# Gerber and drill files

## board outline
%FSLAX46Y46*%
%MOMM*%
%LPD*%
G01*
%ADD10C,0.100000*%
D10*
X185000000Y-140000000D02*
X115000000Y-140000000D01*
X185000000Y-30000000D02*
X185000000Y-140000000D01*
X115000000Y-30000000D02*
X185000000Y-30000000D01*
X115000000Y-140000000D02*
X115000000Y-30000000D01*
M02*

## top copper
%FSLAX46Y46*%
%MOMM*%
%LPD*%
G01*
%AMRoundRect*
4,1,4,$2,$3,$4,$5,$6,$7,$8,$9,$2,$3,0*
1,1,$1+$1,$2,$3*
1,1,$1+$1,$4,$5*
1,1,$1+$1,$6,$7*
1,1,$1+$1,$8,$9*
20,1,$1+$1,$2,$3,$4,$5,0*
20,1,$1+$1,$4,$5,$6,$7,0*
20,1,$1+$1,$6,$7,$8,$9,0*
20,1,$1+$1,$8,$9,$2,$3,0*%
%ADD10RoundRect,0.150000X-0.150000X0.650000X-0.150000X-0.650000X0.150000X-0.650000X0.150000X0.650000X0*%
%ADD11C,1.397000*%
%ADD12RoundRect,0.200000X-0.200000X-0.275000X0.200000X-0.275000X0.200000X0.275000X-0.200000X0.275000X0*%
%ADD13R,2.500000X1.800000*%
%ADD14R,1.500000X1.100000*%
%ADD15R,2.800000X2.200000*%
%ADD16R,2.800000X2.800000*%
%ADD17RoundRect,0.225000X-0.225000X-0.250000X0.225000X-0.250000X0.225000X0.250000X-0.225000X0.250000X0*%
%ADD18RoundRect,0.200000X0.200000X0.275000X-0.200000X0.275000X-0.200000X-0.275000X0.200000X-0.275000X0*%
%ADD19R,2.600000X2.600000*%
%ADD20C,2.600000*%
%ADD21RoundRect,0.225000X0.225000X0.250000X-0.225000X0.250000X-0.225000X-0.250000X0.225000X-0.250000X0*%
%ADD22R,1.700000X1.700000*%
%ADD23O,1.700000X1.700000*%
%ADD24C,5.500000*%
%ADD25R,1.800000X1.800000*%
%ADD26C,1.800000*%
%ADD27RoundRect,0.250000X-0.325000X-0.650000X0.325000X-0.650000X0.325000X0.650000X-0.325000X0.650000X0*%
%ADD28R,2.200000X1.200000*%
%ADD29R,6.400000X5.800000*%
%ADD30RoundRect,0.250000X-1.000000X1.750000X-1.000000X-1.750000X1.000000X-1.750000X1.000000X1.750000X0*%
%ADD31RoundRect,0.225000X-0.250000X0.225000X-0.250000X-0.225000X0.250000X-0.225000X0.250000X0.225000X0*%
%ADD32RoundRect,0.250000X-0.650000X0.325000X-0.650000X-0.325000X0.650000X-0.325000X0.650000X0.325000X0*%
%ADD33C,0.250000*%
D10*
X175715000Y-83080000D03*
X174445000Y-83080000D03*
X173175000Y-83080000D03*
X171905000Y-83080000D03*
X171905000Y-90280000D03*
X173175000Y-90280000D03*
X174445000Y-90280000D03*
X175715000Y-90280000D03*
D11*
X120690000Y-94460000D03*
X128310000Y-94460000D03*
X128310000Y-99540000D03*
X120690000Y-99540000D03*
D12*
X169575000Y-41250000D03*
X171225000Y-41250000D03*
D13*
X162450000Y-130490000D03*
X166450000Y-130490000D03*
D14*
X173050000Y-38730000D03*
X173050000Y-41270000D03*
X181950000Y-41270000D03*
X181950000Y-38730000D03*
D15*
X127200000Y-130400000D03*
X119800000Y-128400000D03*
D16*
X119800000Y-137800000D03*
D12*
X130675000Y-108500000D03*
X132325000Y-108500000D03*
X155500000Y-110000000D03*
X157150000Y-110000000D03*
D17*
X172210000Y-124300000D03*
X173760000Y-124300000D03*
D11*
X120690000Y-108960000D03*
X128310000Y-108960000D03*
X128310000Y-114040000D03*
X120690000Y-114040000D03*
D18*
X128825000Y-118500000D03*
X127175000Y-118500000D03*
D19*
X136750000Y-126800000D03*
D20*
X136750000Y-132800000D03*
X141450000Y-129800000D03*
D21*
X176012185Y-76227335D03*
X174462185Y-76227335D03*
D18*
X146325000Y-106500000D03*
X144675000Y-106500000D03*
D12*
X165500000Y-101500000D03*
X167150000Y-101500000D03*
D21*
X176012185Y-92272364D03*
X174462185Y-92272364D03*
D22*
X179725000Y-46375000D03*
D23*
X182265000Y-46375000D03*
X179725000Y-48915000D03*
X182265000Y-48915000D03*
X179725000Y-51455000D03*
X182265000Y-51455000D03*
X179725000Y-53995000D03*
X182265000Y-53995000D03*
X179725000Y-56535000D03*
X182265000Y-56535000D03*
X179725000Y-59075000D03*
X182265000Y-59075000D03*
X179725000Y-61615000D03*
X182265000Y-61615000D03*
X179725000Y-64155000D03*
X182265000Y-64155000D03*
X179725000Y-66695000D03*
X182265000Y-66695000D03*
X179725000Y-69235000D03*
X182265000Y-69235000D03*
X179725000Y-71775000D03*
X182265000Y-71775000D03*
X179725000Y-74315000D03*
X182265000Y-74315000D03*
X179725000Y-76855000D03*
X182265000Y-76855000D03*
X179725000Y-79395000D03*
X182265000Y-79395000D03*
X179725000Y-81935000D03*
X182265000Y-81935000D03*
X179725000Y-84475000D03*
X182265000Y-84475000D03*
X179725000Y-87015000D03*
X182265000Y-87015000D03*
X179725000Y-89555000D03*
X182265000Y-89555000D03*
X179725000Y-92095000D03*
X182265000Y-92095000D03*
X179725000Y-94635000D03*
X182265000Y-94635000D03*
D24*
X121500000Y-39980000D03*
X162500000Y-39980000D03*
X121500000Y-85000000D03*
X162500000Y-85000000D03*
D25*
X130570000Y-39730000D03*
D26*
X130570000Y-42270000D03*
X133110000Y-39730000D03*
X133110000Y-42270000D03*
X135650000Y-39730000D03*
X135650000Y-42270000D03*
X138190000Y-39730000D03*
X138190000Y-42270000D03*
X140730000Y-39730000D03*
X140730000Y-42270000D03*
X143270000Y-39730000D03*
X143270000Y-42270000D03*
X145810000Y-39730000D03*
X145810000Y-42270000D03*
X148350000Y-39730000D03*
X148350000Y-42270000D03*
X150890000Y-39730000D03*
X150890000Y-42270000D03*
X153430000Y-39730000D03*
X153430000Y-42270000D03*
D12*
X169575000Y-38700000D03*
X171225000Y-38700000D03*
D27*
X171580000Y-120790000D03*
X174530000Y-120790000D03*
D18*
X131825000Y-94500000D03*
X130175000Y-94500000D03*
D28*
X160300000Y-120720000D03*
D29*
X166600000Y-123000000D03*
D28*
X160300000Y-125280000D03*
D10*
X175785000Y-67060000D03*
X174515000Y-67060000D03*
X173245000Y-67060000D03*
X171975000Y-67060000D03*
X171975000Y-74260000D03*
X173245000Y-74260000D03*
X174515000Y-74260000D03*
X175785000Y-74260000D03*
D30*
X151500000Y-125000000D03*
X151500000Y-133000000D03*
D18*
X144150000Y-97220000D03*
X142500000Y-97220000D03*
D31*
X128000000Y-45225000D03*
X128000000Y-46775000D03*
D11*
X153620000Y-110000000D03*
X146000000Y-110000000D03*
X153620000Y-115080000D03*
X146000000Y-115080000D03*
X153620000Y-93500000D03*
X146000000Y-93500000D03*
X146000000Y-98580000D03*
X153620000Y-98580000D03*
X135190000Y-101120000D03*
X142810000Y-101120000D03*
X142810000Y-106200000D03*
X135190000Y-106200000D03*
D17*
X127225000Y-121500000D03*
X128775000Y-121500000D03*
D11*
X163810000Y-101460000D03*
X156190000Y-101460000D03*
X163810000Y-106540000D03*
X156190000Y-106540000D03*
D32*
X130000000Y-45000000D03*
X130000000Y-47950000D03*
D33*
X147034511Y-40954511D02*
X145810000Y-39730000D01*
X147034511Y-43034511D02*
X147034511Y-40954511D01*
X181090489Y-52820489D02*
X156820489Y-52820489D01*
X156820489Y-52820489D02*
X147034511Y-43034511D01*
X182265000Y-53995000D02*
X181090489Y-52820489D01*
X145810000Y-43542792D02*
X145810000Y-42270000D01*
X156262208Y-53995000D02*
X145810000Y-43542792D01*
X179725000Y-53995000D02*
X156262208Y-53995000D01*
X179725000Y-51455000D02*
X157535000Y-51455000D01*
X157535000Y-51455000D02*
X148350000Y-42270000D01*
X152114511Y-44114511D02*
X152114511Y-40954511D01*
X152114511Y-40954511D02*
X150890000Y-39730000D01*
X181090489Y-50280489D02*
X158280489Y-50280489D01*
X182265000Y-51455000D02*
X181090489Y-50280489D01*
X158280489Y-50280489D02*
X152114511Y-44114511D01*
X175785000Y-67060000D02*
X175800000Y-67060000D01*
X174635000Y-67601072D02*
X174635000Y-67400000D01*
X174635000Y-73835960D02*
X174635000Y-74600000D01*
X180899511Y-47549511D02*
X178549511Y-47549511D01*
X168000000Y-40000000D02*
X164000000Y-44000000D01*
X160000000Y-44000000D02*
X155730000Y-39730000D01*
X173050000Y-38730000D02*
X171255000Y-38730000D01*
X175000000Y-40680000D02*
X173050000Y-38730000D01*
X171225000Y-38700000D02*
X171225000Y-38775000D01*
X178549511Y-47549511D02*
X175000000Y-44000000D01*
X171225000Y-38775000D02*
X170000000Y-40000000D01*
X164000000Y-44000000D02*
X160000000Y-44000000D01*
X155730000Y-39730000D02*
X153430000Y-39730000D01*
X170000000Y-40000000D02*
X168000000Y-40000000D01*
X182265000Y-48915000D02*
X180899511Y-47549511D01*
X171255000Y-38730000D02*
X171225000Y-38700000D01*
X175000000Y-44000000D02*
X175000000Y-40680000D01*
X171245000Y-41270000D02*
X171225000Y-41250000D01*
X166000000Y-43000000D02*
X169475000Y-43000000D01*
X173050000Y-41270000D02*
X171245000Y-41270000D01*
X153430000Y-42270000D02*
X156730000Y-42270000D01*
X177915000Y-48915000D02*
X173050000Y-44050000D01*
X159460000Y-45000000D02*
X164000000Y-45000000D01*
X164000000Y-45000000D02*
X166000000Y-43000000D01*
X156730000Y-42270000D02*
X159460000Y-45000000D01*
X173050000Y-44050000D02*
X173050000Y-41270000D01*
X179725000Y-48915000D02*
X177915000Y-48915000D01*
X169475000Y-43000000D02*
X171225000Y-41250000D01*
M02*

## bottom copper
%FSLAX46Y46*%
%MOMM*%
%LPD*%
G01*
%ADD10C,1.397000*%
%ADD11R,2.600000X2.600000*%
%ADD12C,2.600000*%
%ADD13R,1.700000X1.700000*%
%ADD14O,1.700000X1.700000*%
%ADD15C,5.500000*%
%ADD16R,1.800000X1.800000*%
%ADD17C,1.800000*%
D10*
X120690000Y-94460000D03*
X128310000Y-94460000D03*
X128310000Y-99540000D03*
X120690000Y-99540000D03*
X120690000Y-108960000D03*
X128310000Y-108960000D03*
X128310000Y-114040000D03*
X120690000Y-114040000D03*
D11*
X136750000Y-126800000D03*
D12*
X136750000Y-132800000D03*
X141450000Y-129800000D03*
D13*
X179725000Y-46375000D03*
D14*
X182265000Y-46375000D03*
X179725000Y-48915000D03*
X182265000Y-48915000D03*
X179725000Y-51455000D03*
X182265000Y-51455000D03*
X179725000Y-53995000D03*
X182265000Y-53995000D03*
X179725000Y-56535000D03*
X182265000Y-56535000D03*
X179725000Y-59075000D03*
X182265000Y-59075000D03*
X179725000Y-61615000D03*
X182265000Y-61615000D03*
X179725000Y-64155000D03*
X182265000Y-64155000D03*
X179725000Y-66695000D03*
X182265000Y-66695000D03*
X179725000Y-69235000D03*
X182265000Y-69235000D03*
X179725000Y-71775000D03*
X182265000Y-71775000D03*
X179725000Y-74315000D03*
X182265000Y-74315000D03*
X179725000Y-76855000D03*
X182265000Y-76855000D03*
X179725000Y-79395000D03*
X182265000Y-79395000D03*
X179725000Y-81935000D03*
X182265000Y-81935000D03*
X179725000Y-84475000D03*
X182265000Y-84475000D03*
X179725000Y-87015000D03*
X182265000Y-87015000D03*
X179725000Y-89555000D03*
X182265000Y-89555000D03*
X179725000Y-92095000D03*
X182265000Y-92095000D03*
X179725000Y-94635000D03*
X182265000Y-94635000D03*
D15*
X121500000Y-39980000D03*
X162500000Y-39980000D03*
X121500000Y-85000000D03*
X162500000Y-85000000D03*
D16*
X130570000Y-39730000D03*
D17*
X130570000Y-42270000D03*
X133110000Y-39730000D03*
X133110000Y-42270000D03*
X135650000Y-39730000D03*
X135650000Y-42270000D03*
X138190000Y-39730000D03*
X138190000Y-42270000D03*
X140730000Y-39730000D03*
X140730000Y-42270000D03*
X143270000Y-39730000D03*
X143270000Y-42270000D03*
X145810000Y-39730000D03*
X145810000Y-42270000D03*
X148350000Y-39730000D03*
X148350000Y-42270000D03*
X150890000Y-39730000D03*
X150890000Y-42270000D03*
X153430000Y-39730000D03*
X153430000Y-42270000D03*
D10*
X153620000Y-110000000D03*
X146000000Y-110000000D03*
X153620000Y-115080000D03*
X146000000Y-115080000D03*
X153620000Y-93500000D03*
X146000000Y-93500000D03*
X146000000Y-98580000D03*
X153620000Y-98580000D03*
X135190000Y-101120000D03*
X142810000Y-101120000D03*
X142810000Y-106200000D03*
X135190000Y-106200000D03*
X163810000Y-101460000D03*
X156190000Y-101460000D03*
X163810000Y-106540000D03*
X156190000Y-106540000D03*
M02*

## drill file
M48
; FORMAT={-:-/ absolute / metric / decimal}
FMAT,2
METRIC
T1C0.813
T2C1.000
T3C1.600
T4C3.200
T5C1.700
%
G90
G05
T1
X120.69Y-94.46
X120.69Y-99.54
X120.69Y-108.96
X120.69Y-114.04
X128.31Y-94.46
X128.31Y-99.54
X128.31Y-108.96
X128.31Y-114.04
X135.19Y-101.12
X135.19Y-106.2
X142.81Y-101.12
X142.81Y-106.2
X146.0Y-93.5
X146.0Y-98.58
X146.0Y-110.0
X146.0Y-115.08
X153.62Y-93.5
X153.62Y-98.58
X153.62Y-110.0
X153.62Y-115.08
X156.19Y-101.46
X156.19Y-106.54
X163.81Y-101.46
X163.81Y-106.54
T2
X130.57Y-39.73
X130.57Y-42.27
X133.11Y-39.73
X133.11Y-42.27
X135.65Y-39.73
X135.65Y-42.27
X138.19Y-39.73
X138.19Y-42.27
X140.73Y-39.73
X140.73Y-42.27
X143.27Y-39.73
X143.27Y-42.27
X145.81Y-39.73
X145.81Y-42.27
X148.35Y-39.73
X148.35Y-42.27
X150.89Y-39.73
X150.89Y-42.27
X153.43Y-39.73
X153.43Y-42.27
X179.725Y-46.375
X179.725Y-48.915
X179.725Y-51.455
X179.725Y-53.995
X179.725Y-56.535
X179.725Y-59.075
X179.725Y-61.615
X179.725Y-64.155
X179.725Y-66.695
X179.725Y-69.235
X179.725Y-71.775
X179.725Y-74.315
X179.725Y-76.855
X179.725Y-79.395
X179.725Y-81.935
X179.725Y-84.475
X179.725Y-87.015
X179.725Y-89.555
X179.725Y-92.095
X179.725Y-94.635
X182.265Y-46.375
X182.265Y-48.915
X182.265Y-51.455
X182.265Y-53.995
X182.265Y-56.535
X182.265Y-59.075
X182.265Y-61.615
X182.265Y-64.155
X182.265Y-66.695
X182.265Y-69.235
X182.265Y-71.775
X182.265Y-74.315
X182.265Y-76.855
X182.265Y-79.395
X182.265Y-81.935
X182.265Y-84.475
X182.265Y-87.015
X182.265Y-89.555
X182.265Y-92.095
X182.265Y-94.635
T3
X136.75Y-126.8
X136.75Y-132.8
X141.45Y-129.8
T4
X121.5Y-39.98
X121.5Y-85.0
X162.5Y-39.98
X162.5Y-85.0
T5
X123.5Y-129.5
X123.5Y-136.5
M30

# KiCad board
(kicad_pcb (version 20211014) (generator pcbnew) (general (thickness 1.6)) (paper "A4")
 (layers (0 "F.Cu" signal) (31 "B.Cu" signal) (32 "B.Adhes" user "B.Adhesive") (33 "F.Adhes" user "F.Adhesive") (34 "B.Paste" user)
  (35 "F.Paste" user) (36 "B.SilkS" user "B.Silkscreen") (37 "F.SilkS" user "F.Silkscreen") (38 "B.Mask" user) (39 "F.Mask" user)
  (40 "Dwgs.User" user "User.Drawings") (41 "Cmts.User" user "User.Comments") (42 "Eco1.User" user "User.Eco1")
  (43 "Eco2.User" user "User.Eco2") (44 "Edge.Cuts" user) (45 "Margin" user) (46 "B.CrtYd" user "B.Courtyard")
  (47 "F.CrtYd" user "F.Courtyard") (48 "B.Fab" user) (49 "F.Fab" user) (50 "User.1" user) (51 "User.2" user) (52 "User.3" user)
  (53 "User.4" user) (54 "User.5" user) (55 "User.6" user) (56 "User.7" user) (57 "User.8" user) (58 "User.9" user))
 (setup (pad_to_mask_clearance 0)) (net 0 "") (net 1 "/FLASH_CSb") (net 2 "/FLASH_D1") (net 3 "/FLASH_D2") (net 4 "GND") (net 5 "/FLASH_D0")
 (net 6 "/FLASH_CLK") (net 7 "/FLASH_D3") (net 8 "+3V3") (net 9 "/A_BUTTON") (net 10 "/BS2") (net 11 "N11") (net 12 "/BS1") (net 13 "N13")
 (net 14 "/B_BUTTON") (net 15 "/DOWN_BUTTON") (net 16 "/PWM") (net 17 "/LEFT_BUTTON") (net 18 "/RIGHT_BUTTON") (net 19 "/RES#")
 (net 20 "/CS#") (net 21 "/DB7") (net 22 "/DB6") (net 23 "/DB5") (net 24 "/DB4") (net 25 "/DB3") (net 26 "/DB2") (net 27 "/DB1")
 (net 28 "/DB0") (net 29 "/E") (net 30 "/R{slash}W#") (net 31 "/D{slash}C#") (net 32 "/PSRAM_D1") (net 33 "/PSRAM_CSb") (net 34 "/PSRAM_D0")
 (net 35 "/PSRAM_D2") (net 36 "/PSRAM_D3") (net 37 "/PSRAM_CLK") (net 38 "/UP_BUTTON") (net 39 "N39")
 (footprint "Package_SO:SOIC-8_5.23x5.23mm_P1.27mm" (layer "F.Cu") (at 173.81 86.68 -90)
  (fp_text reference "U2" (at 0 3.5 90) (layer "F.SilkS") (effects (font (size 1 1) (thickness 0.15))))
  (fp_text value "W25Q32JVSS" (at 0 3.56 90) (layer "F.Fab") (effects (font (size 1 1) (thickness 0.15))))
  (pad "1" smd roundrect (at -3.6 -1.905 270) (size 1.6 0.6) (layers "F.Cu" "F.Paste" "F.Mask") (roundrect_rratio 0.25) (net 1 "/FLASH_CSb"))
  (pad "2" smd roundrect (at -3.6 -0.635 270) (size 1.6 0.6) (layers "F.Cu" "F.Paste" "F.Mask") (roundrect_rratio 0.25) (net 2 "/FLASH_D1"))
  (pad "3" smd roundrect (at -3.6 0.635 270) (size 1.6 0.6) (layers "F.Cu" "F.Paste" "F.Mask") (roundrect_rratio 0.25) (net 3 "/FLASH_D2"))
  (pad "4" smd roundrect (at -3.6 1.905 270) (size 1.6 0.6) (layers "F.Cu" "F.Paste" "F.Mask") (roundrect_rratio 0.25) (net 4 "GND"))
  (pad "5" smd roundrect (at 3.6 1.905 270) (size 1.6 0.6) (layers "F.Cu" "F.Paste" "F.Mask") (roundrect_rratio 0.25) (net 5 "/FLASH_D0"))
  (pad "6" smd roundrect (at 3.6 0.635 270) (size 1.6 0.6) (layers "F.Cu" "F.Paste" "F.Mask") (roundrect_rratio 0.25) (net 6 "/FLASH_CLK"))
  (pad "7" smd roundrect (at 3.6 -0.635 270) (size 1.6 0.6) (layers "F.Cu" "F.Paste" "F.Mask") (roundrect_rratio 0.25) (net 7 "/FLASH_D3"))
  (pad "8" smd roundrect (at 3.6 -1.905 270) (size 1.6 0.6) (layers "F.Cu" "F.Paste" "F.Mask") (roundrect_rratio 0.25) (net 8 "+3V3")))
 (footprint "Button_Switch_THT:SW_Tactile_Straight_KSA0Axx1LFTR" (layer "F.Cu") (at 120.69 94.46)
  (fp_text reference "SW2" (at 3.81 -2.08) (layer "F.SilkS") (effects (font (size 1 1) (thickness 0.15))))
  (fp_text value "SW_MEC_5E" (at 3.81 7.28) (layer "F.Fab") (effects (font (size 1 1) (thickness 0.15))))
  (pad "1" thru_hole circle (at 0 0) (size 1.397 1.397) (drill 0.8128) (layers *.Cu *.Mask) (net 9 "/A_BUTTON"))
  (pad "1" thru_hole circle (at 7.62 0) (size 1.397 1.397) (drill 0.8128) (layers *.Cu *.Mask) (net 9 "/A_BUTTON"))
  (pad "2" thru_hole circle (at 7.62 5.08) (size 1.397 1.397) (drill 0.8128) (layers *.Cu *.Mask) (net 9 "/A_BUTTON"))
  (pad "2" thru_hole circle (at 0 5.08) (size 1.397 1.397) (drill 0.8128) (layers *.Cu *.Mask) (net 9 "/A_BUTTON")))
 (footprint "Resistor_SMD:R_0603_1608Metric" (layer "F.Cu") (at 170.4 41.25)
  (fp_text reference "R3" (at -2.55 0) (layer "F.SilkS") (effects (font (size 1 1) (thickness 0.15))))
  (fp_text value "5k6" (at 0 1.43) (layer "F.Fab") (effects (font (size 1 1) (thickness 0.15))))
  (pad "1" smd roundrect (at -0.825 0) (size 0.8 0.95) (layers "F.Cu" "F.Paste" "F.Mask") (roundrect_rratio 0.25) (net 4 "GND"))
  (pad "2" smd roundrect (at 0.825 0) (size 0.8 0.95) (layers "F.Cu" "F.Paste" "F.Mask") (roundrect_rratio 0.25) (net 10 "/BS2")))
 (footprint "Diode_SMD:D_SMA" (layer "F.Cu") (at 164.45 130.49)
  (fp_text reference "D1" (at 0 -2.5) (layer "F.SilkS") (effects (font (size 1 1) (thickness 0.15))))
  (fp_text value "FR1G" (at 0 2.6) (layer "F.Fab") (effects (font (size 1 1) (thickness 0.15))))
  (pad "1" smd rect (at -2 0) (size 2.5 1.8) (layers "F.Cu" "F.Paste" "F.Mask") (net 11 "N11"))
  (pad "2" smd rect (at 2 0) (size 2.5 1.8) (layers "F.Cu" "F.Paste" "F.Mask") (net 8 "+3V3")))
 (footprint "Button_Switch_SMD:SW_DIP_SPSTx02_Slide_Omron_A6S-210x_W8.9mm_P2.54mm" (layer "F.Cu") (at 177.5 40)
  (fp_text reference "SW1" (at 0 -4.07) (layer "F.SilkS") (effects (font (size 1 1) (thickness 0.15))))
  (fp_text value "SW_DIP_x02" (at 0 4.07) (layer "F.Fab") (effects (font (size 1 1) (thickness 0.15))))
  (pad "1" smd rect (at -4.45 -1.27) (size 1.5 1.1) (layers "F.Cu" "F.Paste" "F.Mask") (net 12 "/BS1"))
  (pad "2" smd rect (at -4.45 1.27) (size 1.5 1.1) (layers "F.Cu" "F.Paste" "F.Mask") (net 10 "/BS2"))
  (pad "3" smd rect (at 4.45 1.27) (size 1.5 1.1) (layers "F.Cu" "F.Paste" "F.Mask") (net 8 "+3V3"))
  (pad "4" smd rect (at 4.45 -1.27) (size 1.5 1.1) (layers "F.Cu" "F.Paste" "F.Mask") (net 8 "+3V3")))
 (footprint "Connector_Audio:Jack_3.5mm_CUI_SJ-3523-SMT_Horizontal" (layer "F.Cu") (at 123.5 132)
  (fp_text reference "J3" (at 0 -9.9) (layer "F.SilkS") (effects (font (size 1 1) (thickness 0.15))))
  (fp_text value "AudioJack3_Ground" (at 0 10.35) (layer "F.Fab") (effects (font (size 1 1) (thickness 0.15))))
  (pad "" np_thru_hole circle (at 0 4.5) (size 1.7 1.7) (drill 1.7) (layers *.Cu *.Mask))
  (pad "" np_thru_hole circle (at 0 -2.5) (size 1.7 1.7) (drill 1.7) (layers *.Cu *.Mask))
  (pad "R" smd rect (at 3.7 -1.6) (size 2.8 2.2) (layers "F.Cu" "F.Paste" "F.Mask") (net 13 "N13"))
  (pad "S" smd rect (at -3.7 -3.6) (size 2.8 2.2) (layers "F.Cu" "F.Paste" "F.Mask") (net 4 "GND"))
  (pad "T" smd rect (at -3.7 5.8) (size 2.8 2.8) (layers "F.Cu" "F.Paste" "F.Mask") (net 13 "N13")))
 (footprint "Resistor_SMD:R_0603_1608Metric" (layer "F.Cu") (at 131.5 108.5)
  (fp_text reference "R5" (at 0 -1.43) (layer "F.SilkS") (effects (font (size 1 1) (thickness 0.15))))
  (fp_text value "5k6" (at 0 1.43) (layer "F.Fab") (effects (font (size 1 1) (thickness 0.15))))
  (pad "1" smd roundrect (at -0.825 0) (size 0.8 0.95) (layers "F.Cu" "F.Paste" "F.Mask") (roundrect_rratio 0.25) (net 4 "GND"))
  (pad "2" smd roundrect (at 0.825 0) (size 0.8 0.95) (layers "F.Cu" "F.Paste" "F.Mask") (roundrect_rratio 0.25) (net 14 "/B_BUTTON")))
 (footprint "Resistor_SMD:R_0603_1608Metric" (layer "F.Cu") (at 156.325 110)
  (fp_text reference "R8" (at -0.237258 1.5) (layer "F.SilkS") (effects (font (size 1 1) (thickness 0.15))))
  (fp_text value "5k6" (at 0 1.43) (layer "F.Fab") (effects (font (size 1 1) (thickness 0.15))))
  (pad "1" smd roundrect (at -0.825 0) (size 0.8 0.95) (layers "F.Cu" "F.Paste" "F.Mask") (roundrect_rratio 0.25) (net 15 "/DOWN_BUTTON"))
  (pad "2" smd roundrect (at 0.825 0) (size 0.8 0.95) (layers "F.Cu" "F.Paste" "F.Mask") (roundrect_rratio 0.25) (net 4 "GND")))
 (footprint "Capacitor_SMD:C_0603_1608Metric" (layer "F.Cu") (at 172.985 124.3)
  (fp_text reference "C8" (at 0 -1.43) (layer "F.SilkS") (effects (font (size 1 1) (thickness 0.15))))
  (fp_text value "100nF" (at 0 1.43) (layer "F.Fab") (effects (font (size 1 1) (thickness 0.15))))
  (pad "1" smd roundrect (at -0.775 0) (size 0.9 0.95) (layers "F.Cu" "F.Paste" "F.Mask") (roundrect_rratio 0.25) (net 8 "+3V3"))
  (pad "2" smd roundrect (at 0.775 0) (size 0.9 0.95) (layers "F.Cu" "F.Paste" "F.Mask") (roundrect_rratio 0.25) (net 4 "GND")))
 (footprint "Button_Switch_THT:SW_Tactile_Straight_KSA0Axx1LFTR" (layer "F.Cu") (at 120.69 108.96)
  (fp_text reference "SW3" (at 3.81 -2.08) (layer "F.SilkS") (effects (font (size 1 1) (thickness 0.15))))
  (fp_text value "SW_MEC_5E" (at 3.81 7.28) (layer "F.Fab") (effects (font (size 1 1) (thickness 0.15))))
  (pad "1" thru_hole circle (at 0 0) (size 1.397 1.397) (drill 0.8128) (layers *.Cu *.Mask) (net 14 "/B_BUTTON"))
  (pad "1" thru_hole circle (at 7.62 0) (size 1.397 1.397) (drill 0.8128) (layers *.Cu *.Mask) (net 14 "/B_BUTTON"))
  (pad "2" thru_hole circle (at 7.62 5.08) (size 1.397 1.397) (drill 0.8128) (layers *.Cu *.Mask) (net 14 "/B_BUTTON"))
  (pad "2" thru_hole circle (at 0 5.08) (size 1.397 1.397) (drill 0.8128) (layers *.Cu *.Mask) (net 14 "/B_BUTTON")))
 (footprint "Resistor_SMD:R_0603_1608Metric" (layer "F.Cu") (at 128 118.5 180)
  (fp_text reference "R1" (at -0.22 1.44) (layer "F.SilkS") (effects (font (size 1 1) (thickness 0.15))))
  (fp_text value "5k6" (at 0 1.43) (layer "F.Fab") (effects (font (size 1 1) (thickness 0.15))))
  (pad "1" smd roundrect (at -0.825 0 180) (size 0.8 0.95) (layers "F.Cu" "F.Paste" "F.Mask") (roundrect_rratio 0.25) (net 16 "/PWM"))
  (pad "2" smd roundrect (at 0.825 0 180) (size 0.8 0.95) (layers "F.Cu" "F.Paste" "F.Mask") (roundrect_rratio 0.25) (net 13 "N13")))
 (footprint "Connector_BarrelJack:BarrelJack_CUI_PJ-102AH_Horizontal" (layer "F.Cu") (at 136.75 126.8)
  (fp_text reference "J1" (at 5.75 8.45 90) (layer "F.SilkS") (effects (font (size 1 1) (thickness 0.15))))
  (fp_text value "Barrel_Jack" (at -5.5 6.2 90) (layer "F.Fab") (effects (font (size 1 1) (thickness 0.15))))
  (pad "1" thru_hole rect (at 0 0) (size 2.6 2.6) (drill 1.6) (layers *.Cu *.Mask) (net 11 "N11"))
  (pad "2" thru_hole circle (at 0 6) (size 2.6 2.6) (drill 1.6) (layers *.Cu *.Mask) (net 4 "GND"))
  (pad "3" thru_hole circle (at 4.7 3) (size 2.6 2.6) (drill 1.6) (layers *.Cu *.Mask)))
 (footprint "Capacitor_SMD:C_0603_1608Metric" (layer "F.Cu") (at 175.237185 76.227335 180)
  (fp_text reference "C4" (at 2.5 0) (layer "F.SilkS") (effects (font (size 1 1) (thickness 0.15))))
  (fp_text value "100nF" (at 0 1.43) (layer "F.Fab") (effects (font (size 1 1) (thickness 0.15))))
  (pad "1" smd roundrect (at -0.775 0 180) (size 0.9 0.95) (layers "F.Cu" "F.Paste" "F.Mask") (roundrect_rratio 0.25) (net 8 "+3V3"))
  (pad "2" smd roundrect (at 0.775 0 180) (size 0.9 0.95) (layers "F.Cu" "F.Paste" "F.Mask") (roundrect_rratio 0.25) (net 4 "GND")))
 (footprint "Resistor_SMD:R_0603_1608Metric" (layer "F.Cu") (at 145.5 106.5 180)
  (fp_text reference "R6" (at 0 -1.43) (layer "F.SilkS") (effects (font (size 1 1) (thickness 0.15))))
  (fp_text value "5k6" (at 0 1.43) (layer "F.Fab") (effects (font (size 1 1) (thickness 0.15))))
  (pad "1" smd roundrect (at -0.825 0 180) (size 0.8 0.95) (layers "F.Cu" "F.Paste" "F.Mask") (roundrect_rratio 0.25) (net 4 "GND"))
  (pad "2" smd roundrect (at 0.825 0 180) (size 0.8 0.95) (layers "F.Cu" "F.Paste" "F.Mask") (roundrect_rratio 0.25) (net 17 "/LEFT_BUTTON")))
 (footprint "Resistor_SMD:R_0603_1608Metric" (layer "F.Cu") (at 166.325 101.5)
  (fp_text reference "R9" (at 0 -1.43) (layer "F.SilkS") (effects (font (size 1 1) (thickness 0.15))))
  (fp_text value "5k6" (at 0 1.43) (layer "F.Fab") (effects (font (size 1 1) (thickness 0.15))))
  (pad "1" smd roundrect (at -0.825 0) (size 0.8 0.95) (layers "F.Cu" "F.Paste" "F.Mask") (roundrect_rratio 0.25) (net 4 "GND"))
  (pad "2" smd roundrect (at 0.825 0) (size 0.8 0.95) (layers "F.Cu" "F.Paste" "F.Mask") (roundrect_rratio 0.25) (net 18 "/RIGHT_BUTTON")))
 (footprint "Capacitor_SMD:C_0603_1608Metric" (layer "F.Cu") (at 175.237185 92.272364 180)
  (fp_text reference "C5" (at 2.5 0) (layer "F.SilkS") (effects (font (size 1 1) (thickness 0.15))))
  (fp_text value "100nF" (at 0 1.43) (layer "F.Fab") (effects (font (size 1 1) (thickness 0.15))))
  (pad "1" smd roundrect (at -0.775 0 180) (size 0.9 0.95) (layers "F.Cu" "F.Paste" "F.Mask") (roundrect_rratio 0.25) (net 8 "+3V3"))
  (pad "2" smd roundrect (at 0.775 0 180) (size 0.9 0.95) (layers "F.Cu" "F.Paste" "F.Mask") (roundrect_rratio 0.25) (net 4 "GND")))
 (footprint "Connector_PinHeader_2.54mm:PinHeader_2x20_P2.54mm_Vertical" (layer "F.Cu") (at 179.725 46.375)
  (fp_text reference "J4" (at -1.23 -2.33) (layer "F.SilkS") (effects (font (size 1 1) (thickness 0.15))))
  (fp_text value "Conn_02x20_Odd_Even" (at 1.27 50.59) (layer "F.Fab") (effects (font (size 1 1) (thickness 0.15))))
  (pad "1" thru_hole rect (at 0 0) (size 1.7 1.7) (drill 1) (layers *.Cu *.Mask) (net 4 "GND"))
  (pad "2" thru_hole oval (at 2.54 0) (size 1.7 1.7) (drill 1) (layers *.Cu *.Mask) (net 4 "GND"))
  (pad "3" thru_hole oval (at 0 2.54) (size 1.7 1.7) (drill 1) (layers *.Cu *.Mask) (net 10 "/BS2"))
  (pad "4" thru_hole oval (at 2.54 2.54) (size 1.7 1.7) (drill 1) (layers *.Cu *.Mask) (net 12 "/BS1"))
  (pad "5" thru_hole oval (at 0 5.08) (size 1.7 1.7) (drill 1) (layers *.Cu *.Mask) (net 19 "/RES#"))
  (pad "6" thru_hole oval (at 2.54 5.08) (size 1.7 1.7) (drill 1) (layers *.Cu *.Mask) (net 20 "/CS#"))
  (pad "7" thru_hole oval (at 0 7.62) (size 1.7 1.7) (drill 1) (layers *.Cu *.Mask) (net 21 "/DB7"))
  (pad "8" thru_hole oval (at 2.54 7.62) (size 1.7 1.7) (drill 1) (layers *.Cu *.Mask) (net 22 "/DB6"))
  (pad "9" thru_hole oval (at 0 10.16) (size 1.7 1.7) (drill 1) (layers *.Cu *.Mask) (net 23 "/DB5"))
  (pad "10" thru_hole oval (at 2.54 10.16) (size 1.7 1.7) (drill 1) (layers *.Cu *.Mask) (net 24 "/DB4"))
  (pad "11" thru_hole oval (at 0 12.7) (size 1.7 1.7) (drill 1) (layers *.Cu *.Mask) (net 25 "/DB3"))
  (pad "12" thru_hole oval (at 2.54 12.7) (size 1.7 1.7) (drill 1) (layers *.Cu *.Mask) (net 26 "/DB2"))
  (pad "13" thru_hole oval (at 0 15.24) (size 1.7 1.7) (drill 1) (layers *.Cu *.Mask) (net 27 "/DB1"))
  (pad "14" thru_hole oval (at 2.54 15.24) (size 1.7 1.7) (drill 1) (layers *.Cu *.Mask) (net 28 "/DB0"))
  (pad "15" thru_hole oval (at 0 17.78) (size 1.7 1.7) (drill 1) (layers *.Cu *.Mask) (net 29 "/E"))
  (pad "16" thru_hole oval (at 2.54 17.78) (size 1.7 1.7) (drill 1) (layers *.Cu *.Mask) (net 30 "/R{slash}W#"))
  (pad "17" thru_hole oval (at 0 20.32) (size 1.7 1.7) (drill 1) (layers *.Cu *.Mask) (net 16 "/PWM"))
  (pad "18" thru_hole oval (at 2.54 20.32) (size 1.7 1.7) (drill 1) (layers *.Cu *.Mask) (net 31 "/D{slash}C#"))
  (pad "19" thru_hole oval (at 0 22.86) (size 1.7 1.7) (drill 1) (layers *.Cu *.Mask) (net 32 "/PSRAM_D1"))
  (pad "20" thru_hole oval (at 2.54 22.86) (size 1.7 1.7) (drill 1) (layers *.Cu *.Mask) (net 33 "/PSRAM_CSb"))
  (pad "21" thru_hole oval (at 0 25.4) (size 1.7 1.7) (drill 1) (layers *.Cu *.Mask) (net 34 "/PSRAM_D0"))
  (pad "22" thru_hole oval (at 2.54 25.4) (size 1.7 1.7) (drill 1) (layers *.Cu *.Mask) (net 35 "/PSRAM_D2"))
  (pad "23" thru_hole oval (at 0 27.94) (size 1.7 1.7) (drill 1) (layers *.Cu *.Mask) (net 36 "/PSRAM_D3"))
  (pad "24" thru_hole oval (at 2.54 27.94) (size 1.7 1.7) (drill 1) (layers *.Cu *.Mask) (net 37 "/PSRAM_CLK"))
  (pad "25" thru_hole oval (at 0 30.48) (size 1.7 1.7) (drill 1) (layers *.Cu *.Mask) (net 9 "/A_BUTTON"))
  (pad "26" thru_hole oval (at 2.54 30.48) (size 1.7 1.7) (drill 1) (layers *.Cu *.Mask) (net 14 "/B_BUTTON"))
  (pad "27" thru_hole oval (at 0 33.02) (size 1.7 1.7) (drill 1) (layers *.Cu *.Mask) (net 17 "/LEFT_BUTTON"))
  (pad "28" thru_hole oval (at 2.54 33.02) (size 1.7 1.7) (drill 1) (layers *.Cu *.Mask) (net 15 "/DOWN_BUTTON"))
  (pad "29" thru_hole oval (at 0 35.56) (size 1.7 1.7) (drill 1) (layers *.Cu *.Mask) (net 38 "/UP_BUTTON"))
  (pad "30" thru_hole oval (at 2.54 35.56) (size 1.7 1.7) (drill 1) (layers *.Cu *.Mask) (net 18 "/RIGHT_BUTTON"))
  (pad "31" thru_hole oval (at 0 38.1) (size 1.7 1.7) (drill 1) (layers *.Cu *.Mask) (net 2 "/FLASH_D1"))
  (pad "32" thru_hole oval (at 2.54 38.1) (size 1.7 1.7) (drill 1) (layers *.Cu *.Mask) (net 1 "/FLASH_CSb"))
  (pad "33" thru_hole oval (at 0 40.64) (size 1.7 1.7) (drill 1) (layers *.Cu *.Mask) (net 5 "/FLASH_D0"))
  (pad "34" thru_hole oval (at 2.54 40.64) (size 1.7 1.7) (drill 1) (layers *.Cu *.Mask) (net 3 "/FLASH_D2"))
  (pad "35" thru_hole oval (at 0 43.18) (size 1.7 1.7) (drill 1) (layers *.Cu *.Mask) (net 7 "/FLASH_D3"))
  (pad "36" thru_hole oval (at 2.54 43.18) (size 1.7 1.7) (drill 1) (layers *.Cu *.Mask) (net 6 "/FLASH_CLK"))
  (pad "37" thru_hole oval (at 0 45.72) (size 1.7 1.7) (drill 1) (layers *.Cu *.Mask) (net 4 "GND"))
  (pad "38" thru_hole oval (at 2.54 45.72) (size 1.7 1.7) (drill 1) (layers *.Cu *.Mask) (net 4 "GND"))
  (pad "39" thru_hole oval (at 0 48.26) (size 1.7 1.7) (drill 1) (layers *.Cu *.Mask) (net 4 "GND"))
  (pad "40" thru_hole oval (at 2.54 48.26) (size 1.7 1.7) (drill 1) (layers *.Cu *.Mask) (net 4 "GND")))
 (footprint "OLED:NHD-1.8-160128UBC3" (layer "F.Cu") (at 142 41)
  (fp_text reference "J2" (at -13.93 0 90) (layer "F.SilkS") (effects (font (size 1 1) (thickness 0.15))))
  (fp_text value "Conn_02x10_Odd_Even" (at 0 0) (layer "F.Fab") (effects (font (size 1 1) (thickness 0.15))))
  (pad "0" thru_hole circle (at -20.5 -1.02) (size 5.5 5.5) (drill 3.2) (layers *.Cu *.Mask))
  (pad "0" thru_hole circle (at 20.5 -1.02) (size 5.5 5.5) (drill 3.2) (layers *.Cu *.Mask))
  (pad "0" thru_hole circle (at -20.5 44) (size 5.5 5.5) (drill 3.2) (layers *.Cu *.Mask))
  (pad "0" thru_hole circle (at 20.5 44) (size 5.5 5.5) (drill 3.2) (layers *.Cu *.Mask))
  (pad "1" thru_hole rect (at -11.43 -1.27) (size 1.8 1.8) (drill 1) (layers *.Cu *.Mask) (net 4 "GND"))
  (pad "2" thru_hole circle (at -11.43 1.27) (size 1.8 1.8) (drill 1) (layers *.Cu *.Mask) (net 8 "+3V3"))
  (pad "3" thru_hole circle (at -8.89 -1.27) (size 1.8 1.8) (drill 1) (layers *.Cu *.Mask) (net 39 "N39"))
  (pad "4" thru_hole circle (at -8.89 1.27) (size 1.8 1.8) (drill 1) (layers *.Cu *.Mask) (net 31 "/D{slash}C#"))
  (pad "5" thru_hole circle (at -6.35 -1.27) (size 1.8 1.8) (drill 1) (layers *.Cu *.Mask) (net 30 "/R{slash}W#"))
  (pad "6" thru_hole circle (at -6.35 1.27) (size 1.8 1.8) (drill 1) (layers *.Cu *.Mask) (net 29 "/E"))
  (pad "7" thru_hole circle (at -3.81 -1.27) (size 1.8 1.8) (drill 1) (layers *.Cu *.Mask) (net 28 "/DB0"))
  (pad "8" thru_hole circle (at -3.81 1.27) (size 1.8 1.8) (drill 1) (layers *.Cu *.Mask) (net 27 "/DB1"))
  (pad "9" thru_hole circle (at -1.27 -1.27) (size 1.8 1.8) (drill 1) (layers *.Cu *.Mask) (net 26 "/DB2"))
  (pad "10" thru_hole circle (at -1.27 1.27) (size 1.8 1.8) (drill 1) (layers *.Cu *.Mask) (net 25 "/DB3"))
  (pad "11" thru_hole circle (at 1.27 -1.27) (size 1.8 1.8) (drill 1) (layers *.Cu *.Mask) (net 24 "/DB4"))
  (pad "12" thru_hole circle (at 1.27 1.27) (size 1.8 1.8) (drill 1) (layers *.Cu *.Mask) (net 23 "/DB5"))
  (pad "13" thru_hole circle (at 3.81 -1.27) (size 1.8 1.8) (drill 1) (layers *.Cu *.Mask) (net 22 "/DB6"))
  (pad "14" thru_hole circle (at 3.81 1.27) (size 1.8 1.8) (drill 1) (layers *.Cu *.Mask) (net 21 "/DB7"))
  (pad "15" thru_hole circle (at 6.35 -1.27) (size 1.8 1.8) (drill 1) (layers *.Cu *.Mask) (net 4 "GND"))
  (pad "16" thru_hole circle (at 6.35 1.27) (size 1.8 1.8) (drill 1) (layers *.Cu *.Mask) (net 19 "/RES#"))
  (pad "17" thru_hole circle (at 8.89 -1.27) (size 1.8 1.8) (drill 1) (layers *.Cu *.Mask) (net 20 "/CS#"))
  (pad "18" thru_hole circle (at 8.89 1.27) (size 1.8 1.8) (drill 1) (layers *.Cu *.Mask) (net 4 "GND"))
  (pad "19" thru_hole circle (at 11.43 -1.27) (size 1.8 1.8) (drill 1) (layers *.Cu *.Mask) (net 12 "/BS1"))
  (pad "20" thru_hole circle (at 11.43 1.27) (size 1.8 1.8) (drill 1) (layers *.Cu *.Mask) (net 10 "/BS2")))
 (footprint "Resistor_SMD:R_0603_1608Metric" (layer "F.Cu") (at 170.4 38.7)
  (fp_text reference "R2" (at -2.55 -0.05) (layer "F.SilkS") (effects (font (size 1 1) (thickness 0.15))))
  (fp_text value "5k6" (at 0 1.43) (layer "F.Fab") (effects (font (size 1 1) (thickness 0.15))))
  (pad "1" smd roundrect (at -0.825 0) (size 0.8 0.95) (layers "F.Cu" "F.Paste" "F.Mask") (roundrect_rratio 0.25) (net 4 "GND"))
  (pad "2" smd roundrect (at 0.825 0) (size 0.8 0.95) (layers "F.Cu" "F.Paste" "F.Mask") (roundrect_rratio 0.25) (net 12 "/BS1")))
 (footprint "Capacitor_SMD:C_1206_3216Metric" (layer "F.Cu") (at 173.055 120.79)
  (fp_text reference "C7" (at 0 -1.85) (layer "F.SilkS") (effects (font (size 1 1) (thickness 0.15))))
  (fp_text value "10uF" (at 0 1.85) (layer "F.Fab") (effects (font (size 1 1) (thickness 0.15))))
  (pad "1" smd roundrect (at -1.475 0) (size 1.15 1.8) (layers "F.Cu" "F.Paste" "F.Mask") (roundrect_rratio 0.217391) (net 8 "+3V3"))
  (pad "2" smd roundrect (at 1.475 0) (size 1.15 1.8) (layers "F.Cu" "F.Paste" "F.Mask") (roundrect_rratio 0.217391) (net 4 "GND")))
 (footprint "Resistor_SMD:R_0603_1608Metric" (layer "F.Cu") (at 131 94.5 180)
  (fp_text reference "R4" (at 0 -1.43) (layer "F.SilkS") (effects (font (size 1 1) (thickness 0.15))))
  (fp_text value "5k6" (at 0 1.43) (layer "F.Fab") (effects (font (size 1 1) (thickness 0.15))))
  (pad "1" smd roundrect (at -0.825 0 180) (size 0.8 0.95) (layers "F.Cu" "F.Paste" "F.Mask") (roundrect_rratio 0.25) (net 4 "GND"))
  (pad "2" smd roundrect (at 0.825 0 180) (size 0.8 0.95) (layers "F.Cu" "F.Paste" "F.Mask") (roundrect_rratio 0.25) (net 9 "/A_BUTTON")))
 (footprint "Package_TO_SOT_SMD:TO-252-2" (layer "F.Cu") (at 164.5 123)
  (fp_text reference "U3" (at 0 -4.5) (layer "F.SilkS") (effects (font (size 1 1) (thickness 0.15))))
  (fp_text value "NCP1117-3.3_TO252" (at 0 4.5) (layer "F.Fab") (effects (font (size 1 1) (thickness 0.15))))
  (pad "" smd rect (at 3.775 1.525) (size 3.05 2.75) (layers "F.Paste"))
  (pad "" smd rect (at 0.425 -1.525) (size 3.05 2.75) (layers "F.Paste"))
  (pad "" smd rect (at 3.775 -1.525) (size 3.05 2.75) (layers "F.Paste"))
  (pad "" smd rect (at 0.425 1.525) (size 3.05 2.75) (layers "F.Paste"))
  (pad "1" smd rect (at -4.2 -2.28) (size 2.2 1.2) (layers "F.Cu" "F.Paste" "F.Mask") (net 4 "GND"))
  (pad "2" smd rect (at 2.1 0) (size 6.4 5.8) (layers "F.Cu" "F.Mask") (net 8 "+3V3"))
  (pad "3" smd rect (at -4.2 2.28) (size 2.2 1.2) (layers "F.Cu" "F.Paste" "F.Mask") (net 11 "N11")))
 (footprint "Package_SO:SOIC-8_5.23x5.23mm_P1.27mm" (layer "F.Cu") (at 173.88 70.66 -90)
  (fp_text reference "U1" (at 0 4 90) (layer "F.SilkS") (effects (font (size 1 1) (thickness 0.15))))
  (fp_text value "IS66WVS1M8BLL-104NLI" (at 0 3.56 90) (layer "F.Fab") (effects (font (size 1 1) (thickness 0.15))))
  (pad "1" smd roundrect (at -3.6 -1.905 270) (size 1.6 0.6) (layers "F.Cu" "F.Paste" "F.Mask") (roundrect_rratio 0.25)
   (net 33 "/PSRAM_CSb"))
  (pad "2" smd roundrect (at -3.6 -0.635 270) (size 1.6 0.6) (layers "F.Cu" "F.Paste" "F.Mask") (roundrect_rratio 0.25) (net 32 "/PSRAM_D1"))
  (pad "3" smd roundrect (at -3.6 0.635 270) (size 1.6 0.6) (layers "F.Cu" "F.Paste" "F.Mask") (roundrect_rratio 0.25) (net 35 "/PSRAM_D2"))
  (pad "4" smd roundrect (at -3.6 1.905 270) (size 1.6 0.6) (layers "F.Cu" "F.Paste" "F.Mask") (roundrect_rratio 0.25) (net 4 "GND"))
  (pad "5" smd roundrect (at 3.6 1.905 270) (size 1.6 0.6) (layers "F.Cu" "F.Paste" "F.Mask") (roundrect_rratio 0.25) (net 34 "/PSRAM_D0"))
  (pad "6" smd roundrect (at 3.6 0.635 270) (size 1.6 0.6) (layers "F.Cu" "F.Paste" "F.Mask") (roundrect_rratio 0.25) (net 37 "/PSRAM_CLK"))
  (pad "7" smd roundrect (at 3.6 -0.635 270) (size 1.6 0.6) (layers "F.Cu" "F.Paste" "F.Mask") (roundrect_rratio 0.25) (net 36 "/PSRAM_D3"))
  (pad "8" smd roundrect (at 3.6 -1.905 270) (size 1.6 0.6) (layers "F.Cu" "F.Paste" "F.Mask") (roundrect_rratio 0.25) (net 8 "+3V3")))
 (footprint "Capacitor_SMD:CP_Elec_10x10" (layer "F.Cu") (at 151.5 129 -90)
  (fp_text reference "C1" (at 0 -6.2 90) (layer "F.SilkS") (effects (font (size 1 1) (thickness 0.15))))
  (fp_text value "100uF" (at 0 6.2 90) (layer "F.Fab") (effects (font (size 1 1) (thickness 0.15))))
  (pad "1" smd roundrect (at -4 0 270) (size 4 2.5) (layers "F.Cu" "F.Paste" "F.Mask") (roundrect_rratio 0.1) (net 11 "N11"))
  (pad "2" smd roundrect (at 4 0 270) (size 4 2.5) (layers "F.Cu" "F.Paste" "F.Mask") (roundrect_rratio 0.1) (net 4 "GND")))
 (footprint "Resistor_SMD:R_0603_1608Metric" (layer "F.Cu") (at 143.325 97.22 180)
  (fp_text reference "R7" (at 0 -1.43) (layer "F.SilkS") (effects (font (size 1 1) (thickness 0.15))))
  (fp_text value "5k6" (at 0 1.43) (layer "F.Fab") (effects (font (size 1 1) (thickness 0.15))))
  (pad "1" smd roundrect (at -0.825 0 180) (size 0.8 0.95) (layers "F.Cu" "F.Paste" "F.Mask") (roundrect_rratio 0.25) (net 4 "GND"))
  (pad "2" smd roundrect (at 0.825 0 180) (size 0.8 0.95) (layers "F.Cu" "F.Paste" "F.Mask") (roundrect_rratio 0.25) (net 38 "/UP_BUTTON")))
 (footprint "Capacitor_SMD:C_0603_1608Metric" (layer "F.Cu") (at 128 46 -90)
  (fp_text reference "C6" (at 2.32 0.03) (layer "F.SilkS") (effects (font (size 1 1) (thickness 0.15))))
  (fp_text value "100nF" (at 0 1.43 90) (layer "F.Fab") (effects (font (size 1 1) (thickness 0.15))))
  (pad "1" smd roundrect (at -0.775 0 270) (size 0.9 0.95) (layers "F.Cu" "F.Paste" "F.Mask") (roundrect_rratio 0.25) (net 8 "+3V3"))
  (pad "2" smd roundrect (at 0.775 0 270) (size 0.9 0.95) (layers "F.Cu" "F.Paste" "F.Mask") (roundrect_rratio 0.25) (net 4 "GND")))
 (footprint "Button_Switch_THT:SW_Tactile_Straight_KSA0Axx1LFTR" (layer "F.Cu") (at 146 110)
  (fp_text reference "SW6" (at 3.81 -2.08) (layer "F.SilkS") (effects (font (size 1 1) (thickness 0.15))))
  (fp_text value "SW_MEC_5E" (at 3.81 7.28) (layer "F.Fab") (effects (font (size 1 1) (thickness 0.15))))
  (pad "1" thru_hole circle (at 7.62 0) (size 1.397 1.397) (drill 0.8128) (layers *.Cu *.Mask) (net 15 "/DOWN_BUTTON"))
  (pad "1" thru_hole circle (at 0 0) (size 1.397 1.397) (drill 0.8128) (layers *.Cu *.Mask) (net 15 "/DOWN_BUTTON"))
  (pad "2" thru_hole circle (at 7.62 5.08) (size 1.397 1.397) (drill 0.8128) (layers *.Cu *.Mask) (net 15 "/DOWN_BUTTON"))
  (pad "2" thru_hole circle (at 0 5.08) (size 1.397 1.397) (drill 0.8128) (layers *.Cu *.Mask) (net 15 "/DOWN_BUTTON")))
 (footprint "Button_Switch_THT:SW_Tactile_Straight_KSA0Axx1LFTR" (layer "F.Cu") (at 146 93.5)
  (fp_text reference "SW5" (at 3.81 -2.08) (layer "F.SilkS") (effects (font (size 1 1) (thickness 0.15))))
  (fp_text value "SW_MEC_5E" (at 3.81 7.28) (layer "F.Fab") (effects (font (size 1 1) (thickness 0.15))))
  (pad "1" thru_hole circle (at 7.62 0) (size 1.397 1.397) (drill 0.8128) (layers *.Cu *.Mask) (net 38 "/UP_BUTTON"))
  (pad "1" thru_hole circle (at 0 0) (size 1.397 1.397) (drill 0.8128) (layers *.Cu *.Mask) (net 38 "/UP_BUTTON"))
  (pad "2" thru_hole circle (at 0 5.08) (size 1.397 1.397) (drill 0.8128) (layers *.Cu *.Mask) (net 38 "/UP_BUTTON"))
  (pad "2" thru_hole circle (at 7.62 5.08) (size 1.397 1.397) (drill 0.8128) (layers *.Cu *.Mask) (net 38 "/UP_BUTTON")))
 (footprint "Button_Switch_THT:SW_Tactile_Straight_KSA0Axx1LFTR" (layer "F.Cu") (at 135.19 101.12)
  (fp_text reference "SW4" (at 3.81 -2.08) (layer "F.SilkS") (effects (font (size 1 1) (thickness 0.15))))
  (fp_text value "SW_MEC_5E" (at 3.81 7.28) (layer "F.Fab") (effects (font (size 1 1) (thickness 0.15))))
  (pad "1" thru_hole circle (at 0 0) (size 1.397 1.397) (drill 0.8128) (layers *.Cu *.Mask) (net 17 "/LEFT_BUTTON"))
  (pad "1" thru_hole circle (at 7.62 0) (size 1.397 1.397) (drill 0.8128) (layers *.Cu *.Mask) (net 17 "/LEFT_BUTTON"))
  (pad "2" thru_hole circle (at 7.62 5.08) (size 1.397 1.397) (drill 0.8128) (layers *.Cu *.Mask) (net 17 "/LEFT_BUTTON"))
  (pad "2" thru_hole circle (at 0 5.08) (size 1.397 1.397) (drill 0.8128) (layers *.Cu *.Mask) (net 17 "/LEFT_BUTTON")))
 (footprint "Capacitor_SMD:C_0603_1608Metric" (layer "F.Cu") (at 128 121.5)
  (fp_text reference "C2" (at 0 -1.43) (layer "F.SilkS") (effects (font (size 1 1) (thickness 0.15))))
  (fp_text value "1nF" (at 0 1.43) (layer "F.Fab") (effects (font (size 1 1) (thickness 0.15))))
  (pad "1" smd roundrect (at -0.775 0) (size 0.9 0.95) (layers "F.Cu" "F.Paste" "F.Mask") (roundrect_rratio 0.25) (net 13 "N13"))
  (pad "2" smd roundrect (at 0.775 0) (size 0.9 0.95) (layers "F.Cu" "F.Paste" "F.Mask") (roundrect_rratio 0.25) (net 4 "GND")))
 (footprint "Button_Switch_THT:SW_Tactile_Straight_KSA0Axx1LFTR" (layer "F.Cu") (at 156.19 101.46)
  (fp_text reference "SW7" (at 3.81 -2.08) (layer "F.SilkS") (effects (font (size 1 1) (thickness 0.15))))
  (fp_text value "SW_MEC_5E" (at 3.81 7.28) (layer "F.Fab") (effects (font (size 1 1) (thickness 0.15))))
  (pad "1" thru_hole circle (at 7.62 0) (size 1.397 1.397) (drill 0.8128) (layers *.Cu *.Mask) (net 18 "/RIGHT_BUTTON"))
  (pad "1" thru_hole circle (at 0 0) (size 1.397 1.397) (drill 0.8128) (layers *.Cu *.Mask) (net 18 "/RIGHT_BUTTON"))
  (pad "2" thru_hole circle (at 7.62 5.08) (size 1.397 1.397) (drill 0.8128) (layers *.Cu *.Mask) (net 18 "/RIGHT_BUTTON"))
  (pad "2" thru_hole circle (at 0 5.08) (size 1.397 1.397) (drill 0.8128) (layers *.Cu *.Mask) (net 18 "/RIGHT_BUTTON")))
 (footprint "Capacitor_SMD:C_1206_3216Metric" (layer "F.Cu") (at 130 46.475 -90)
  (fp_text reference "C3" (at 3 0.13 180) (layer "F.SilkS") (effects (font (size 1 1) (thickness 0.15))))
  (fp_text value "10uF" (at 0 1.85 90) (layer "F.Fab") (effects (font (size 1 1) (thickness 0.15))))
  (pad "1" smd roundrect (at -1.475 0 270) (size 1.15 1.8) (layers "F.Cu" "F.Paste" "F.Mask") (roundrect_rratio 0.217391) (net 8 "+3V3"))
  (pad "2" smd roundrect (at 1.475 0 270) (size 1.15 1.8) (layers "F.Cu" "F.Paste" "F.Mask") (roundrect_rratio 0.217391) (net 4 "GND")))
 (gr_line (start 185 140) (end 115 140) (layer "Edge.Cuts") (width 0.1))
 (gr_line (start 185 30) (end 185 140) (layer "Edge.Cuts") (width 0.1))
 (gr_line (start 115 30) (end 185 30) (layer "Edge.Cuts") (width 0.1))
 (gr_line (start 115 140) (end 115 30) (layer "Edge.Cuts") (width 0.1))
 (segment (start 147.034511 40.954511) (end 145.81 39.73) (width 0.25) (layer "F.Cu") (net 22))
 (segment (start 147.034511 43.034511) (end 147.034511 40.954511) (width 0.25) (layer "F.Cu") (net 22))
 (segment (start 181.090489 52.820489) (end 156.820489 52.820489) (width 0.25) (layer "F.Cu") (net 22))
 (segment (start 156.820489 52.820489) (end 147.034511 43.034511) (width 0.25) (layer "F.Cu") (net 22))
 (segment (start 182.265 53.995) (end 181.090489 52.820489) (width 0.25) (layer "F.Cu") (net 22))
 (segment (start 145.81 43.542792) (end 145.81 42.27) (width 0.25) (layer "F.Cu") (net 21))
 (segment (start 156.262208 53.995) (end 145.81 43.542792) (width 0.25) (layer "F.Cu") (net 21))
 (segment (start 179.725 53.995) (end 156.262208 53.995) (width 0.25) (layer "F.Cu") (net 21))
 (segment (start 179.725 51.455) (end 157.535 51.455) (width 0.25) (layer "F.Cu") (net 19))
 (segment (start 157.535 51.455) (end 148.35 42.27) (width 0.25) (layer "F.Cu") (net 19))
 (segment (start 152.114511 44.114511) (end 152.114511 40.954511) (width 0.25) (layer "F.Cu") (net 20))
 (segment (start 152.114511 40.954511) (end 150.89 39.73) (width 0.25) (layer "F.Cu") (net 20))
 (segment (start 181.090489 50.280489) (end 158.280489 50.280489) (width 0.25) (layer "F.Cu") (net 20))
 (segment (start 182.265 51.455) (end 181.090489 50.280489) (width 0.25) (layer "F.Cu") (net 20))
 (segment (start 158.280489 50.280489) (end 152.114511 44.114511) (width 0.25) (layer "F.Cu") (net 20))
 (segment (start 175.785 67.06) (end 175.8 67.06) (width 0.25) (layer "F.Cu") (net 33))
 (segment (start 174.635 67.601072) (end 174.635 67.4) (width 0.25) (layer "F.Cu") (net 32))
 (segment (start 174.635 73.83596) (end 174.635 74.6) (width 0.25) (layer "F.Cu") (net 36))
 (segment (start 180.899511 47.549511) (end 178.549511 47.549511) (width 0.25) (layer "F.Cu") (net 12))
 (segment (start 168 40) (end 164 44) (width 0.25) (layer "F.Cu") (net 12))
 (segment (start 160 44) (end 155.73 39.73) (width 0.25) (layer "F.Cu") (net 12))
 (segment (start 173.05 38.73) (end 171.255 38.73) (width 0.25) (layer "F.Cu") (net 12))
 (segment (start 175 40.68) (end 173.05 38.73) (width 0.25) (layer "F.Cu") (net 12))
 (segment (start 171.225 38.7) (end 171.225 38.775) (width 0.25) (layer "F.Cu") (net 12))
 (segment (start 178.549511 47.549511) (end 175 44) (width 0.25) (layer "F.Cu") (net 12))
 (segment (start 171.225 38.775) (end 170 40) (width 0.25) (layer "F.Cu") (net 12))
 (segment (start 164 44) (end 160 44) (width 0.25) (layer "F.Cu") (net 12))
 (segment (start 155.73 39.73) (end 153.43 39.73) (width 0.25) (layer "F.Cu") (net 12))
 (segment (start 170 40) (end 168 40) (width 0.25) (layer "F.Cu") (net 12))
 (segment (start 182.265 48.915) (end 180.899511 47.549511) (width 0.25) (layer "F.Cu") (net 12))
 (segment (start 171.255 38.73) (end 171.225 38.7) (width 0.25) (layer "F.Cu") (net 12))
 (segment (start 175 44) (end 175 40.68) (width 0.25) (layer "F.Cu") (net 12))
 (segment (start 171.245 41.27) (end 171.225 41.25) (width 0.25) (layer "F.Cu") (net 10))
 (segment (start 166 43) (end 169.475 43) (width 0.25) (layer "F.Cu") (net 10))
 (segment (start 173.05 41.27) (end 171.245 41.27) (width 0.25) (layer "F.Cu") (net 10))
 (segment (start 153.43 42.27) (end 156.73 42.27) (width 0.25) (layer "F.Cu") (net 10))
 (segment (start 177.915 48.915) (end 173.05 44.05) (width 0.25) (layer "F.Cu") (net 10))
 (segment (start 159.46 45) (end 164 45) (width 0.25) (layer "F.Cu") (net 10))
 (segment (start 164 45) (end 166 43) (width 0.25) (layer "F.Cu") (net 10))
 (segment (start 156.73 42.27) (end 159.46 45) (width 0.25) (layer "F.Cu") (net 10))
 (segment (start 173.05 44.05) (end 173.05 41.27) (width 0.25) (layer "F.Cu") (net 10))
 (segment (start 179.725 48.915) (end 177.915 48.915) (width 0.25) (layer "F.Cu") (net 10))
 (segment (start 169.475 43) (end 171.225 41.25) (width 0.25) (layer "F.Cu") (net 10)))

